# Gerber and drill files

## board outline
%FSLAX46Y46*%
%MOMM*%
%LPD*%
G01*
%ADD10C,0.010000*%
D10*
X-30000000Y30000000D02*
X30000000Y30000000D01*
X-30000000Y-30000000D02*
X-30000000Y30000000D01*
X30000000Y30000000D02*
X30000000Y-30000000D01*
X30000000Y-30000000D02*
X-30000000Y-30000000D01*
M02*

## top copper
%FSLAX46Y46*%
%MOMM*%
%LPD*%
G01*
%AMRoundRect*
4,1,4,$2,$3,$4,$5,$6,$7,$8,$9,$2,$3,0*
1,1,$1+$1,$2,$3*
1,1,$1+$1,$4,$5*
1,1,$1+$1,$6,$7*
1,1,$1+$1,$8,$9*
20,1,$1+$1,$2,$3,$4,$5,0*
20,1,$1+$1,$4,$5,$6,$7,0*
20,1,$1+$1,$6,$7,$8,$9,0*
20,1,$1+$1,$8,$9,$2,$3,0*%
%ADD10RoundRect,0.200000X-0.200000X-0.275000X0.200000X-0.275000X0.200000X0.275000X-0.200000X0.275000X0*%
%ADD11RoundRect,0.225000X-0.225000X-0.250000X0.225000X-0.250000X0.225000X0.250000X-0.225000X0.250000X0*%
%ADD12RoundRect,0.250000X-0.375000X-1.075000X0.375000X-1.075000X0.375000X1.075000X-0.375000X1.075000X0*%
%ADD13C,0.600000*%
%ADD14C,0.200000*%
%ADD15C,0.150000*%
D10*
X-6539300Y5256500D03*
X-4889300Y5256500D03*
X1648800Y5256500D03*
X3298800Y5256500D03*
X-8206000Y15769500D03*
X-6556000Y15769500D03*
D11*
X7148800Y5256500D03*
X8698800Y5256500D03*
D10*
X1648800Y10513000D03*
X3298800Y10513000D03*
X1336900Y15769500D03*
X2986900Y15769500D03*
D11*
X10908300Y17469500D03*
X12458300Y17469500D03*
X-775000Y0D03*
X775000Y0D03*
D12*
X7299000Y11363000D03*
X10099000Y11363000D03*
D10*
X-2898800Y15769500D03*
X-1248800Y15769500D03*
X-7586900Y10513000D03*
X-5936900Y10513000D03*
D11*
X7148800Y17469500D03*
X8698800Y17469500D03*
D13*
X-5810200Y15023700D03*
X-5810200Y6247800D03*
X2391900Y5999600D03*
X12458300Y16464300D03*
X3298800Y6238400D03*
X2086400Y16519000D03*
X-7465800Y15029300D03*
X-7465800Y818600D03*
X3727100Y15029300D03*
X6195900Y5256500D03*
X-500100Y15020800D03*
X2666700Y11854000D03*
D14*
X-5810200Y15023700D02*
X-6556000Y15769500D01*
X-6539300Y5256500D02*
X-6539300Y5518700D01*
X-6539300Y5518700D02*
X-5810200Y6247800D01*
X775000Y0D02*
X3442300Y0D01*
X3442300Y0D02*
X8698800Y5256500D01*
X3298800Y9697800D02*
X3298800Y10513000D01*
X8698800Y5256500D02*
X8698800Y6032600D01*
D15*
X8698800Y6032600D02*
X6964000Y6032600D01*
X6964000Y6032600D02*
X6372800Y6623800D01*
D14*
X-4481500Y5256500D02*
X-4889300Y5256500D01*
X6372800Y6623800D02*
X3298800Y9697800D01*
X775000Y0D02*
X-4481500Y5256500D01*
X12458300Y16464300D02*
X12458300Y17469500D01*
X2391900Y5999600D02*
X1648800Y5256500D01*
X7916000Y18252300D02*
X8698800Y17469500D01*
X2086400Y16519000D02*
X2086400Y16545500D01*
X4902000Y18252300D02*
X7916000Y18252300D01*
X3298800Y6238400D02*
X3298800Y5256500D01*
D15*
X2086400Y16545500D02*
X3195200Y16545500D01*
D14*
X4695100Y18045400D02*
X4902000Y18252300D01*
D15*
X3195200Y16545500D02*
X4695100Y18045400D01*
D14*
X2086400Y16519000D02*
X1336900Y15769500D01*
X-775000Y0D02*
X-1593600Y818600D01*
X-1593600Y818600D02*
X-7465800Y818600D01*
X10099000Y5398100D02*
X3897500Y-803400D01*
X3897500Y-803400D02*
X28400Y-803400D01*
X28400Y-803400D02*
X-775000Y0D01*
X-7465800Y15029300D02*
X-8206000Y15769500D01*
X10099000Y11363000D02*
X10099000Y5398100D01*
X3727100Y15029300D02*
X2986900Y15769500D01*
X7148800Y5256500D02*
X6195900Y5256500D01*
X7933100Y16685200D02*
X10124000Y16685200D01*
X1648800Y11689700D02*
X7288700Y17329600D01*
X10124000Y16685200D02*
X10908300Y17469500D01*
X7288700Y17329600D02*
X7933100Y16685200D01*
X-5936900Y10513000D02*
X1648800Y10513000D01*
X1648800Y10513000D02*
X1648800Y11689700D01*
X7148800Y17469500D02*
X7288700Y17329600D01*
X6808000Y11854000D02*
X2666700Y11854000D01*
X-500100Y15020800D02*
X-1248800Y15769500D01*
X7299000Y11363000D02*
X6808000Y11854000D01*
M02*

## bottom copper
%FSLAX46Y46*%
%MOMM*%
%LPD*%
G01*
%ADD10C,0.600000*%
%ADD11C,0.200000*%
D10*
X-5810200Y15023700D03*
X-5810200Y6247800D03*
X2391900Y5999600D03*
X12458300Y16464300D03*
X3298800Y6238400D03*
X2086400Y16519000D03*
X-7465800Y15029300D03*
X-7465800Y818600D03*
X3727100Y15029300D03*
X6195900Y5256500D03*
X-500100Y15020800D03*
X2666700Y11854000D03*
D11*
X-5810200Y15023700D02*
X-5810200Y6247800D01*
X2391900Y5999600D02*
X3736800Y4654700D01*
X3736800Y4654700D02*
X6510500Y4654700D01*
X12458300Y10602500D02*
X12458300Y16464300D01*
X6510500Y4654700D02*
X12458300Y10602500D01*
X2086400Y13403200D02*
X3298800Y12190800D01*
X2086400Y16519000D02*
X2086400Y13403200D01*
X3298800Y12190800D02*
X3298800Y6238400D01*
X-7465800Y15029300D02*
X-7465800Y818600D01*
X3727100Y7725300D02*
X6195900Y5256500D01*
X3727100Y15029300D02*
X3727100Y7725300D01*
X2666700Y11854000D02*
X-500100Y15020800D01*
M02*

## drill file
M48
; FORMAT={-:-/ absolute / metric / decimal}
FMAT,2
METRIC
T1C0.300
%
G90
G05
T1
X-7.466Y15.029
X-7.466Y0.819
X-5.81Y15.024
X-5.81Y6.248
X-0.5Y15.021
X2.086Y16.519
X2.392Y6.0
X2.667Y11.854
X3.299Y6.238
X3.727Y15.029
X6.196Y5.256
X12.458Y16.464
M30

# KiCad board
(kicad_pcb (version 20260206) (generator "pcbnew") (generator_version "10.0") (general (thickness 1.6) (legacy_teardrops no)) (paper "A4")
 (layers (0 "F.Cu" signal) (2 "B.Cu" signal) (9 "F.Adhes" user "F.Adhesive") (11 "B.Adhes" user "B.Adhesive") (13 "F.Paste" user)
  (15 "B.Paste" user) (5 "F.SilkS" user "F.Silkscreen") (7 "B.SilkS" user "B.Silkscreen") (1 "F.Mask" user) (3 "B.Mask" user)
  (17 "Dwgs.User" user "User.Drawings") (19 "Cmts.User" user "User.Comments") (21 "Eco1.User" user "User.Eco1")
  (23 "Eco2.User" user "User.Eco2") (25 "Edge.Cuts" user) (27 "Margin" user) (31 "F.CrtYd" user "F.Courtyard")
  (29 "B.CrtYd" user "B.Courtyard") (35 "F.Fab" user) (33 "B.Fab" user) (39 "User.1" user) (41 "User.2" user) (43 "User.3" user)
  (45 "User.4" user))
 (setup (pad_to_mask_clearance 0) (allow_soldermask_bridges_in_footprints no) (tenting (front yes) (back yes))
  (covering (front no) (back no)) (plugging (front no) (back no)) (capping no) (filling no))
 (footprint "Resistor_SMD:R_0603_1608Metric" (layer "F.Cu") (at -5.7143 -5.2565)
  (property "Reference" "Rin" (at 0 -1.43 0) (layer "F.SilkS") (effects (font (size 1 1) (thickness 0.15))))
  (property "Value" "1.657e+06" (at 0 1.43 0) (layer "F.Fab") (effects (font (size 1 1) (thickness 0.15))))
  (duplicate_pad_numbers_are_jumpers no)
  (pad "1" smd roundrect (at -0.825 0) (size 0.8 0.95) (layers "F.Cu" "F.Mask" "F.Paste") (roundrect_rratio 0.25) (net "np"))
  (pad "2" smd roundrect (at 0.825 0) (size 0.8 0.95) (layers "F.Cu" "F.Mask" "F.Paste") (roundrect_rratio 0.25) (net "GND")))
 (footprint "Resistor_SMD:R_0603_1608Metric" (layer "F.Cu") (at 2.4738 -5.2565)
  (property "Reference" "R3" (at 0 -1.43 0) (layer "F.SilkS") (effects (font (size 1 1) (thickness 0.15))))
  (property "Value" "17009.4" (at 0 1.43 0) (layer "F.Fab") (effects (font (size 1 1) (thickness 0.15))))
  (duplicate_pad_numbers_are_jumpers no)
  (pad "1" smd roundrect (at -0.825 0) (size 0.8 0.95) (layers "F.Cu" "F.Mask" "F.Paste") (roundrect_rratio 0.25) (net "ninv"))
  (pad "2" smd roundrect (at 0.825 0) (size 0.8 0.95) (layers "F.Cu" "F.Mask" "F.Paste") (roundrect_rratio 0.25) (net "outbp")))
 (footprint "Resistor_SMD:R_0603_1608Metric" (layer "F.Cu") (at -7.381 -15.7695)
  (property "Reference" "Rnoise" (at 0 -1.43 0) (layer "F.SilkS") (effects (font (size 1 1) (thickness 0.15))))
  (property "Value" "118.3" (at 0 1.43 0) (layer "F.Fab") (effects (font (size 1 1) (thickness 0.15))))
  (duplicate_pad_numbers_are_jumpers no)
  (pad "1" smd roundrect (at -0.825 0) (size 0.8 0.95) (layers "F.Cu" "F.Mask" "F.Paste") (roundrect_rratio 0.25) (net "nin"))
  (pad "2" smd roundrect (at 0.825 0) (size 0.8 0.95) (layers "F.Cu" "F.Mask" "F.Paste") (roundrect_rratio 0.25) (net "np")))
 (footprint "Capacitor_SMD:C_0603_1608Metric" (layer "F.Cu") (at 7.9238 -5.2565)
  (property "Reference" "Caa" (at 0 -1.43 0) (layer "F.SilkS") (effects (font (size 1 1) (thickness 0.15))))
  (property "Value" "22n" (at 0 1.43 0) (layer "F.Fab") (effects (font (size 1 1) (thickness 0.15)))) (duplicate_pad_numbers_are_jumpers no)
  (pad "1" smd roundrect (at -0.775 0) (size 0.9 0.95) (layers "F.Cu" "F.Mask" "F.Paste") (roundrect_rratio 0.25) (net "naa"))
  (pad "2" smd roundrect (at 0.775 0) (size 0.9 0.95) (layers "F.Cu" "F.Mask" "F.Paste") (roundrect_rratio 0.25) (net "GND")))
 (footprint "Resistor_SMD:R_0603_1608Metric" (layer "F.Cu") (at 2.4738 -10.513)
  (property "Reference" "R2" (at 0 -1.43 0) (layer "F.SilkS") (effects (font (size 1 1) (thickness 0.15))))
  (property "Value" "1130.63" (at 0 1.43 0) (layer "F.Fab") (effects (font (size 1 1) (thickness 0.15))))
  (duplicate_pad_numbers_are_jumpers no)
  (pad "1" smd roundrect (at -0.825 0) (size 0.8 0.95) (layers "F.Cu" "F.Mask" "F.Paste") (roundrect_rratio 0.25) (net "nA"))
  (pad "2" smd roundrect (at 0.825 0) (size 0.8 0.95) (layers "F.Cu" "F.Mask" "F.Paste") (roundrect_rratio 0.25) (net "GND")))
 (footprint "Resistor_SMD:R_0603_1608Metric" (layer "F.Cu") (at 2.1619 -15.7695)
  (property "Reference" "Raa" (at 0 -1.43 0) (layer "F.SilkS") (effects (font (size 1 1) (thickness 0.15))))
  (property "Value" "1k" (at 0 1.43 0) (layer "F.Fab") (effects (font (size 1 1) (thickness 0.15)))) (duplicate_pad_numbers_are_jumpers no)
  (pad "1" smd roundrect (at -0.825 0) (size 0.8 0.95) (layers "F.Cu" "F.Mask" "F.Paste") (roundrect_rratio 0.25) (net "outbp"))
  (pad "2" smd roundrect (at 0.825 0) (size 0.8 0.95) (layers "F.Cu" "F.Mask" "F.Paste") (roundrect_rratio 0.25) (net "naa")))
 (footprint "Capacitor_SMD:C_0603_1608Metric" (layer "F.Cu") (at 11.6833 -17.4695)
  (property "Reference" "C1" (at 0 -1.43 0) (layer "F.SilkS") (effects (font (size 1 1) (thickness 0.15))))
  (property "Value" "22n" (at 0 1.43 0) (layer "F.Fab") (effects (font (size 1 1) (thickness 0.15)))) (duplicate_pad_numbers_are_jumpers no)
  (pad "1" smd roundrect (at -0.775 0) (size 0.9 0.95) (layers "F.Cu" "F.Mask" "F.Paste") (roundrect_rratio 0.25) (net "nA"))
  (pad "2" smd roundrect (at 0.775 0) (size 0.9 0.95) (layers "F.Cu" "F.Mask" "F.Paste") (roundrect_rratio 0.25) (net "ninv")))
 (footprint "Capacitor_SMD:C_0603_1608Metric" (layer "F.Cu") (at 0 0)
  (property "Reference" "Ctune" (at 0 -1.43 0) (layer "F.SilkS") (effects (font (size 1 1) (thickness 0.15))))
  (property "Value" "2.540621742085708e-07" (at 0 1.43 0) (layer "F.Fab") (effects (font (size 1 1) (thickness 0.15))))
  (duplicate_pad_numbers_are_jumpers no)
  (pad "1" smd roundrect (at -0.775 0) (size 0.9 0.95) (layers "F.Cu" "F.Mask" "F.Paste") (roundrect_rratio 0.25) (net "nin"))
  (pad "2" smd roundrect (at 0.775 0) (size 0.9 0.95) (layers "F.Cu" "F.Mask" "F.Paste") (roundrect_rratio 0.25) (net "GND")))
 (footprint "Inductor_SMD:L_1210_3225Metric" (layer "F.Cu") (at 8.699 -11.363)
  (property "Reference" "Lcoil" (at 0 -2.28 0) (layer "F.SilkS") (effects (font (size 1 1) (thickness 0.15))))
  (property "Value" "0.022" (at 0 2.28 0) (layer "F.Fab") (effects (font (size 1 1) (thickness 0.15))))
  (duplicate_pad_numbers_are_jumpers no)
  (pad "1" smd roundrect (at -1.4 0) (size 1.25 2.65) (layers "F.Cu" "F.Mask" "F.Paste") (roundrect_rratio 0.2) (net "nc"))
  (pad "2" smd roundrect (at 1.4 0) (size 1.25 2.65) (layers "F.Cu" "F.Mask" "F.Paste") (roundrect_rratio 0.2) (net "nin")))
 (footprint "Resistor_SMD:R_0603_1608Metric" (layer "F.Cu") (at -2.0738 -15.7695)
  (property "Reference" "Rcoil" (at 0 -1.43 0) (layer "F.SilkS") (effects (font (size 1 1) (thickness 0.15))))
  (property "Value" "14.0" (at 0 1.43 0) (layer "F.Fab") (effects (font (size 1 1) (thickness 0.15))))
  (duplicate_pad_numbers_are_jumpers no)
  (pad "1" smd roundrect (at -0.825 0) (size 0.8 0.95) (layers "F.Cu" "F.Mask" "F.Paste") (roundrect_rratio 0.25) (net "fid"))
  (pad "2" smd roundrect (at 0.825 0) (size 0.8 0.95) (layers "F.Cu" "F.Mask" "F.Paste") (roundrect_rratio 0.25) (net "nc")))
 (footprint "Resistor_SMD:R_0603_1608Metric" (layer "F.Cu") (at -6.7619 -10.513)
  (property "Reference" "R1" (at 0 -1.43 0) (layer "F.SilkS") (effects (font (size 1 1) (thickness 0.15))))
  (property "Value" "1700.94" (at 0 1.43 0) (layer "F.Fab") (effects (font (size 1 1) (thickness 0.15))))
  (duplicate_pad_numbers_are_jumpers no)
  (pad "1" smd roundrect (at -0.825 0) (size 0.8 0.95) (layers "F.Cu" "F.Mask" "F.Paste") (roundrect_rratio 0.25) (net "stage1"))
  (pad "2" smd roundrect (at 0.825 0) (size 0.8 0.95) (layers "F.Cu" "F.Mask" "F.Paste") (roundrect_rratio 0.25) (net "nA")))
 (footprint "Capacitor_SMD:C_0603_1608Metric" (layer "F.Cu") (at 7.9238 -17.4695)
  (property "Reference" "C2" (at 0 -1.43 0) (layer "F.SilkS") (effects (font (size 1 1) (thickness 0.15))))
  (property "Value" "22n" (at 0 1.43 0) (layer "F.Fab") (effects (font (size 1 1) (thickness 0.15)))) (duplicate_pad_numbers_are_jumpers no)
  (pad "1" smd roundrect (at -0.775 0) (size 0.9 0.95) (layers "F.Cu" "F.Mask" "F.Paste") (roundrect_rratio 0.25) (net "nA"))
  (pad "2" smd roundrect (at 0.775 0) (size 0.9 0.95) (layers "F.Cu" "F.Mask" "F.Paste") (roundrect_rratio 0.25) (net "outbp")))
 (gr_line (start -30 -30) (end 30 -30) (stroke (width 0.01) (type default)) (layer "Edge.Cuts"))
 (gr_line (start -30 30) (end -30 -30) (stroke (width 0.01) (type default)) (layer "Edge.Cuts"))
 (gr_line (start 30 -30) (end 30 30) (stroke (width 0.01) (type default)) (layer "Edge.Cuts"))
 (gr_line (start 30 30) (end -30 30) (stroke (width 0.01) (type default)) (layer "Edge.Cuts"))
 (segment (start -5.8102 -15.0237) (end -6.556 -15.7695) (width 0.2) (layer "F.Cu") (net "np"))
 (segment (start -6.5393 -5.2565) (end -6.5393 -5.5187) (width 0.2) (layer "F.Cu") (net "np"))
 (segment (start -6.5393 -5.5187) (end -5.8102 -6.2478) (width 0.2) (layer "F.Cu") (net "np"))
 (via (at -5.8102 -15.0237) (size 0.6) (drill 0.3) (layers "F.Cu" "B.Cu") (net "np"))
 (via (at -5.8102 -6.2478) (size 0.6) (drill 0.3) (layers "F.Cu" "B.Cu") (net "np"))
 (segment (start -5.8102 -15.0237) (end -5.8102 -6.2478) (width 0.2) (layer "B.Cu") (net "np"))
 (segment (start 0.775 0) (end 3.4423 0) (width 0.2) (layer "F.Cu") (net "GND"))
 (segment (start 3.4423 0) (end 8.6988 -5.2565) (width 0.2) (layer "F.Cu") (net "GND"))
 (segment (start 3.2988 -9.6978) (end 3.2988 -10.513) (width 0.2) (layer "F.Cu") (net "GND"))
 (segment (start 8.6988 -5.2565) (end 8.6988 -6.0326) (width 0.2) (layer "F.Cu") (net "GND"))
 (segment (start 8.6988 -6.0326) (end 6.964 -6.0326) (width 0.15) (layer "F.Cu") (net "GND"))
 (segment (start 6.964 -6.0326) (end 6.3728 -6.6238) (width 0.15) (layer "F.Cu") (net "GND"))
 (segment (start -4.4815 -5.2565) (end -4.8893 -5.2565) (width 0.2) (layer "F.Cu") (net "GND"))
 (segment (start 6.3728 -6.6238) (end 3.2988 -9.6978) (width 0.2) (layer "F.Cu") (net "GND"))
 (segment (start 0.775 0) (end -4.4815 -5.2565) (width 0.2) (layer "F.Cu") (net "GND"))
 (segment (start 12.4583 -16.4643) (end 12.4583 -17.4695) (width 0.2) (layer "F.Cu") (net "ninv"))
 (segment (start 2.3919 -5.9996) (end 1.6488 -5.2565) (width 0.2) (layer "F.Cu") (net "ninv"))
 (via (at 2.3919 -5.9996) (size 0.6) (drill 0.3) (layers "F.Cu" "B.Cu") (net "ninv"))
 (via (at 12.4583 -16.4643) (size 0.6) (drill 0.3) (layers "F.Cu" "B.Cu") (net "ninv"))
 (segment (start 2.3919 -5.9996) (end 3.7368 -4.6547) (width 0.2) (layer "B.Cu") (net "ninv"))
 (segment (start 3.7368 -4.6547) (end 6.5105 -4.6547) (width 0.2) (layer "B.Cu") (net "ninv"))
 (segment (start 12.4583 -10.6025) (end 12.4583 -16.4643) (width 0.2) (layer "B.Cu") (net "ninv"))
 (segment (start 6.5105 -4.6547) (end 12.4583 -10.6025) (width 0.2) (layer "B.Cu") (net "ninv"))
 (segment (start 7.916 -18.2523) (end 8.6988 -17.4695) (width 0.2) (layer "F.Cu") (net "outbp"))
 (segment (start 2.0864 -16.519) (end 2.0864 -16.5455) (width 0.2) (layer "F.Cu") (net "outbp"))
 (segment (start 4.902 -18.2523) (end 7.916 -18.2523) (width 0.2) (layer "F.Cu") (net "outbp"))
 (segment (start 3.2988 -6.2384) (end 3.2988 -5.2565) (width 0.2) (layer "F.Cu") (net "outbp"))
 (segment (start 2.0864 -16.5455) (end 3.1952 -16.5455) (width 0.15) (layer "F.Cu") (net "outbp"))
 (segment (start 4.6951 -18.0454) (end 4.902 -18.2523) (width 0.2) (layer "F.Cu") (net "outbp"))
 (segment (start 3.1952 -16.5455) (end 4.6951 -18.0454) (width 0.15) (layer "F.Cu") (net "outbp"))
 (segment (start 2.0864 -16.519) (end 1.3369 -15.7695) (width 0.2) (layer "F.Cu") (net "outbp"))
 (via (at 3.2988 -6.2384) (size 0.6) (drill 0.3) (layers "F.Cu" "B.Cu") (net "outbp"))
 (via (at 2.0864 -16.519) (size 0.6) (drill 0.3) (layers "F.Cu" "B.Cu") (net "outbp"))
 (segment (start 2.0864 -13.4032) (end 3.2988 -12.1908) (width 0.2) (layer "B.Cu") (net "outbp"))
 (segment (start 2.0864 -16.519) (end 2.0864 -13.4032) (width 0.2) (layer "B.Cu") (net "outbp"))
 (segment (start 3.2988 -12.1908) (end 3.2988 -6.2384) (width 0.2) (layer "B.Cu") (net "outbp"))
 (segment (start -0.775 0) (end -1.5936 -0.8186) (width 0.2) (layer "F.Cu") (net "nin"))
 (segment (start -1.5936 -0.8186) (end -7.4658 -0.8186) (width 0.2) (layer "F.Cu") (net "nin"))
 (segment (start 10.099 -5.3981) (end 3.8975 0.8034) (width 0.2) (layer "F.Cu") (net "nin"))
 (segment (start 3.8975 0.8034) (end 0.0284 0.8034) (width 0.2) (layer "F.Cu") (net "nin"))
 (segment (start 0.0284 0.8034) (end -0.775 0) (width 0.2) (layer "F.Cu") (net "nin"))
 (segment (start -7.4658 -15.0293) (end -8.206 -15.7695) (width 0.2) (layer "F.Cu") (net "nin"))
 (segment (start 10.099 -11.363) (end 10.099 -5.3981) (width 0.2) (layer "F.Cu") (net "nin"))
 (via (at -7.4658 -15.0293) (size 0.6) (drill 0.3) (layers "F.Cu" "B.Cu") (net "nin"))
 (via (at -7.4658 -0.8186) (size 0.6) (drill 0.3) (layers "F.Cu" "B.Cu") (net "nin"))
 (segment (start -7.4658 -15.0293) (end -7.4658 -0.8186) (width 0.2) (layer "B.Cu") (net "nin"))
 (segment (start 3.7271 -15.0293) (end 2.9869 -15.7695) (width 0.2) (layer "F.Cu") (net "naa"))
 (segment (start 7.1488 -5.2565) (end 6.1959 -5.2565) (width 0.2) (layer "F.Cu") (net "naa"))
 (via (at 3.7271 -15.0293) (size 0.6) (drill 0.3) (layers "F.Cu" "B.Cu") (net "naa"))
 (via (at 6.1959 -5.2565) (size 0.6) (drill 0.3) (layers "F.Cu" "B.Cu") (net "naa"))
 (segment (start 3.7271 -7.7253) (end 6.1959 -5.2565) (width 0.2) (layer "B.Cu") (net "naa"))
 (segment (start 3.7271 -15.0293) (end 3.7271 -7.7253) (width 0.2) (layer "B.Cu") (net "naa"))
 (segment (start 7.9331 -16.6852) (end 10.124 -16.6852) (width 0.2) (layer "F.Cu") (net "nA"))
 (segment (start 1.6488 -11.6897) (end 7.2887 -17.3296) (width 0.2) (layer "F.Cu") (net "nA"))
 (segment (start 10.124 -16.6852) (end 10.9083 -17.4695) (width 0.2) (layer "F.Cu") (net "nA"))
 (segment (start 7.2887 -17.3296) (end 7.9331 -16.6852) (width 0.2) (layer "F.Cu") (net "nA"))
 (segment (start -5.9369 -10.513) (end 1.6488 -10.513) (width 0.2) (layer "F.Cu") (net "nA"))
 (segment (start 1.6488 -10.513) (end 1.6488 -11.6897) (width 0.2) (layer "F.Cu") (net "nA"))
 (segment (start 7.1488 -17.4695) (end 7.2887 -17.3296) (width 0.2) (layer "F.Cu") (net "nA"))
 (segment (start 6.808 -11.854) (end 2.6667 -11.854) (width 0.2) (layer "F.Cu") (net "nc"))
 (segment (start -0.5001 -15.0208) (end -1.2488 -15.7695) (width 0.2) (layer "F.Cu") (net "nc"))
 (segment (start 7.299 -11.363) (end 6.808 -11.854) (width 0.2) (layer "F.Cu") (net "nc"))
 (via (at -0.5001 -15.0208) (size 0.6) (drill 0.3) (layers "F.Cu" "B.Cu") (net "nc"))
 (via (at 2.6667 -11.854) (size 0.6) (drill 0.3) (layers "F.Cu" "B.Cu") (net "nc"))
 (segment (start 2.6667 -11.854) (end -0.5001 -15.0208) (width 0.2) (layer "B.Cu") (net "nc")))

